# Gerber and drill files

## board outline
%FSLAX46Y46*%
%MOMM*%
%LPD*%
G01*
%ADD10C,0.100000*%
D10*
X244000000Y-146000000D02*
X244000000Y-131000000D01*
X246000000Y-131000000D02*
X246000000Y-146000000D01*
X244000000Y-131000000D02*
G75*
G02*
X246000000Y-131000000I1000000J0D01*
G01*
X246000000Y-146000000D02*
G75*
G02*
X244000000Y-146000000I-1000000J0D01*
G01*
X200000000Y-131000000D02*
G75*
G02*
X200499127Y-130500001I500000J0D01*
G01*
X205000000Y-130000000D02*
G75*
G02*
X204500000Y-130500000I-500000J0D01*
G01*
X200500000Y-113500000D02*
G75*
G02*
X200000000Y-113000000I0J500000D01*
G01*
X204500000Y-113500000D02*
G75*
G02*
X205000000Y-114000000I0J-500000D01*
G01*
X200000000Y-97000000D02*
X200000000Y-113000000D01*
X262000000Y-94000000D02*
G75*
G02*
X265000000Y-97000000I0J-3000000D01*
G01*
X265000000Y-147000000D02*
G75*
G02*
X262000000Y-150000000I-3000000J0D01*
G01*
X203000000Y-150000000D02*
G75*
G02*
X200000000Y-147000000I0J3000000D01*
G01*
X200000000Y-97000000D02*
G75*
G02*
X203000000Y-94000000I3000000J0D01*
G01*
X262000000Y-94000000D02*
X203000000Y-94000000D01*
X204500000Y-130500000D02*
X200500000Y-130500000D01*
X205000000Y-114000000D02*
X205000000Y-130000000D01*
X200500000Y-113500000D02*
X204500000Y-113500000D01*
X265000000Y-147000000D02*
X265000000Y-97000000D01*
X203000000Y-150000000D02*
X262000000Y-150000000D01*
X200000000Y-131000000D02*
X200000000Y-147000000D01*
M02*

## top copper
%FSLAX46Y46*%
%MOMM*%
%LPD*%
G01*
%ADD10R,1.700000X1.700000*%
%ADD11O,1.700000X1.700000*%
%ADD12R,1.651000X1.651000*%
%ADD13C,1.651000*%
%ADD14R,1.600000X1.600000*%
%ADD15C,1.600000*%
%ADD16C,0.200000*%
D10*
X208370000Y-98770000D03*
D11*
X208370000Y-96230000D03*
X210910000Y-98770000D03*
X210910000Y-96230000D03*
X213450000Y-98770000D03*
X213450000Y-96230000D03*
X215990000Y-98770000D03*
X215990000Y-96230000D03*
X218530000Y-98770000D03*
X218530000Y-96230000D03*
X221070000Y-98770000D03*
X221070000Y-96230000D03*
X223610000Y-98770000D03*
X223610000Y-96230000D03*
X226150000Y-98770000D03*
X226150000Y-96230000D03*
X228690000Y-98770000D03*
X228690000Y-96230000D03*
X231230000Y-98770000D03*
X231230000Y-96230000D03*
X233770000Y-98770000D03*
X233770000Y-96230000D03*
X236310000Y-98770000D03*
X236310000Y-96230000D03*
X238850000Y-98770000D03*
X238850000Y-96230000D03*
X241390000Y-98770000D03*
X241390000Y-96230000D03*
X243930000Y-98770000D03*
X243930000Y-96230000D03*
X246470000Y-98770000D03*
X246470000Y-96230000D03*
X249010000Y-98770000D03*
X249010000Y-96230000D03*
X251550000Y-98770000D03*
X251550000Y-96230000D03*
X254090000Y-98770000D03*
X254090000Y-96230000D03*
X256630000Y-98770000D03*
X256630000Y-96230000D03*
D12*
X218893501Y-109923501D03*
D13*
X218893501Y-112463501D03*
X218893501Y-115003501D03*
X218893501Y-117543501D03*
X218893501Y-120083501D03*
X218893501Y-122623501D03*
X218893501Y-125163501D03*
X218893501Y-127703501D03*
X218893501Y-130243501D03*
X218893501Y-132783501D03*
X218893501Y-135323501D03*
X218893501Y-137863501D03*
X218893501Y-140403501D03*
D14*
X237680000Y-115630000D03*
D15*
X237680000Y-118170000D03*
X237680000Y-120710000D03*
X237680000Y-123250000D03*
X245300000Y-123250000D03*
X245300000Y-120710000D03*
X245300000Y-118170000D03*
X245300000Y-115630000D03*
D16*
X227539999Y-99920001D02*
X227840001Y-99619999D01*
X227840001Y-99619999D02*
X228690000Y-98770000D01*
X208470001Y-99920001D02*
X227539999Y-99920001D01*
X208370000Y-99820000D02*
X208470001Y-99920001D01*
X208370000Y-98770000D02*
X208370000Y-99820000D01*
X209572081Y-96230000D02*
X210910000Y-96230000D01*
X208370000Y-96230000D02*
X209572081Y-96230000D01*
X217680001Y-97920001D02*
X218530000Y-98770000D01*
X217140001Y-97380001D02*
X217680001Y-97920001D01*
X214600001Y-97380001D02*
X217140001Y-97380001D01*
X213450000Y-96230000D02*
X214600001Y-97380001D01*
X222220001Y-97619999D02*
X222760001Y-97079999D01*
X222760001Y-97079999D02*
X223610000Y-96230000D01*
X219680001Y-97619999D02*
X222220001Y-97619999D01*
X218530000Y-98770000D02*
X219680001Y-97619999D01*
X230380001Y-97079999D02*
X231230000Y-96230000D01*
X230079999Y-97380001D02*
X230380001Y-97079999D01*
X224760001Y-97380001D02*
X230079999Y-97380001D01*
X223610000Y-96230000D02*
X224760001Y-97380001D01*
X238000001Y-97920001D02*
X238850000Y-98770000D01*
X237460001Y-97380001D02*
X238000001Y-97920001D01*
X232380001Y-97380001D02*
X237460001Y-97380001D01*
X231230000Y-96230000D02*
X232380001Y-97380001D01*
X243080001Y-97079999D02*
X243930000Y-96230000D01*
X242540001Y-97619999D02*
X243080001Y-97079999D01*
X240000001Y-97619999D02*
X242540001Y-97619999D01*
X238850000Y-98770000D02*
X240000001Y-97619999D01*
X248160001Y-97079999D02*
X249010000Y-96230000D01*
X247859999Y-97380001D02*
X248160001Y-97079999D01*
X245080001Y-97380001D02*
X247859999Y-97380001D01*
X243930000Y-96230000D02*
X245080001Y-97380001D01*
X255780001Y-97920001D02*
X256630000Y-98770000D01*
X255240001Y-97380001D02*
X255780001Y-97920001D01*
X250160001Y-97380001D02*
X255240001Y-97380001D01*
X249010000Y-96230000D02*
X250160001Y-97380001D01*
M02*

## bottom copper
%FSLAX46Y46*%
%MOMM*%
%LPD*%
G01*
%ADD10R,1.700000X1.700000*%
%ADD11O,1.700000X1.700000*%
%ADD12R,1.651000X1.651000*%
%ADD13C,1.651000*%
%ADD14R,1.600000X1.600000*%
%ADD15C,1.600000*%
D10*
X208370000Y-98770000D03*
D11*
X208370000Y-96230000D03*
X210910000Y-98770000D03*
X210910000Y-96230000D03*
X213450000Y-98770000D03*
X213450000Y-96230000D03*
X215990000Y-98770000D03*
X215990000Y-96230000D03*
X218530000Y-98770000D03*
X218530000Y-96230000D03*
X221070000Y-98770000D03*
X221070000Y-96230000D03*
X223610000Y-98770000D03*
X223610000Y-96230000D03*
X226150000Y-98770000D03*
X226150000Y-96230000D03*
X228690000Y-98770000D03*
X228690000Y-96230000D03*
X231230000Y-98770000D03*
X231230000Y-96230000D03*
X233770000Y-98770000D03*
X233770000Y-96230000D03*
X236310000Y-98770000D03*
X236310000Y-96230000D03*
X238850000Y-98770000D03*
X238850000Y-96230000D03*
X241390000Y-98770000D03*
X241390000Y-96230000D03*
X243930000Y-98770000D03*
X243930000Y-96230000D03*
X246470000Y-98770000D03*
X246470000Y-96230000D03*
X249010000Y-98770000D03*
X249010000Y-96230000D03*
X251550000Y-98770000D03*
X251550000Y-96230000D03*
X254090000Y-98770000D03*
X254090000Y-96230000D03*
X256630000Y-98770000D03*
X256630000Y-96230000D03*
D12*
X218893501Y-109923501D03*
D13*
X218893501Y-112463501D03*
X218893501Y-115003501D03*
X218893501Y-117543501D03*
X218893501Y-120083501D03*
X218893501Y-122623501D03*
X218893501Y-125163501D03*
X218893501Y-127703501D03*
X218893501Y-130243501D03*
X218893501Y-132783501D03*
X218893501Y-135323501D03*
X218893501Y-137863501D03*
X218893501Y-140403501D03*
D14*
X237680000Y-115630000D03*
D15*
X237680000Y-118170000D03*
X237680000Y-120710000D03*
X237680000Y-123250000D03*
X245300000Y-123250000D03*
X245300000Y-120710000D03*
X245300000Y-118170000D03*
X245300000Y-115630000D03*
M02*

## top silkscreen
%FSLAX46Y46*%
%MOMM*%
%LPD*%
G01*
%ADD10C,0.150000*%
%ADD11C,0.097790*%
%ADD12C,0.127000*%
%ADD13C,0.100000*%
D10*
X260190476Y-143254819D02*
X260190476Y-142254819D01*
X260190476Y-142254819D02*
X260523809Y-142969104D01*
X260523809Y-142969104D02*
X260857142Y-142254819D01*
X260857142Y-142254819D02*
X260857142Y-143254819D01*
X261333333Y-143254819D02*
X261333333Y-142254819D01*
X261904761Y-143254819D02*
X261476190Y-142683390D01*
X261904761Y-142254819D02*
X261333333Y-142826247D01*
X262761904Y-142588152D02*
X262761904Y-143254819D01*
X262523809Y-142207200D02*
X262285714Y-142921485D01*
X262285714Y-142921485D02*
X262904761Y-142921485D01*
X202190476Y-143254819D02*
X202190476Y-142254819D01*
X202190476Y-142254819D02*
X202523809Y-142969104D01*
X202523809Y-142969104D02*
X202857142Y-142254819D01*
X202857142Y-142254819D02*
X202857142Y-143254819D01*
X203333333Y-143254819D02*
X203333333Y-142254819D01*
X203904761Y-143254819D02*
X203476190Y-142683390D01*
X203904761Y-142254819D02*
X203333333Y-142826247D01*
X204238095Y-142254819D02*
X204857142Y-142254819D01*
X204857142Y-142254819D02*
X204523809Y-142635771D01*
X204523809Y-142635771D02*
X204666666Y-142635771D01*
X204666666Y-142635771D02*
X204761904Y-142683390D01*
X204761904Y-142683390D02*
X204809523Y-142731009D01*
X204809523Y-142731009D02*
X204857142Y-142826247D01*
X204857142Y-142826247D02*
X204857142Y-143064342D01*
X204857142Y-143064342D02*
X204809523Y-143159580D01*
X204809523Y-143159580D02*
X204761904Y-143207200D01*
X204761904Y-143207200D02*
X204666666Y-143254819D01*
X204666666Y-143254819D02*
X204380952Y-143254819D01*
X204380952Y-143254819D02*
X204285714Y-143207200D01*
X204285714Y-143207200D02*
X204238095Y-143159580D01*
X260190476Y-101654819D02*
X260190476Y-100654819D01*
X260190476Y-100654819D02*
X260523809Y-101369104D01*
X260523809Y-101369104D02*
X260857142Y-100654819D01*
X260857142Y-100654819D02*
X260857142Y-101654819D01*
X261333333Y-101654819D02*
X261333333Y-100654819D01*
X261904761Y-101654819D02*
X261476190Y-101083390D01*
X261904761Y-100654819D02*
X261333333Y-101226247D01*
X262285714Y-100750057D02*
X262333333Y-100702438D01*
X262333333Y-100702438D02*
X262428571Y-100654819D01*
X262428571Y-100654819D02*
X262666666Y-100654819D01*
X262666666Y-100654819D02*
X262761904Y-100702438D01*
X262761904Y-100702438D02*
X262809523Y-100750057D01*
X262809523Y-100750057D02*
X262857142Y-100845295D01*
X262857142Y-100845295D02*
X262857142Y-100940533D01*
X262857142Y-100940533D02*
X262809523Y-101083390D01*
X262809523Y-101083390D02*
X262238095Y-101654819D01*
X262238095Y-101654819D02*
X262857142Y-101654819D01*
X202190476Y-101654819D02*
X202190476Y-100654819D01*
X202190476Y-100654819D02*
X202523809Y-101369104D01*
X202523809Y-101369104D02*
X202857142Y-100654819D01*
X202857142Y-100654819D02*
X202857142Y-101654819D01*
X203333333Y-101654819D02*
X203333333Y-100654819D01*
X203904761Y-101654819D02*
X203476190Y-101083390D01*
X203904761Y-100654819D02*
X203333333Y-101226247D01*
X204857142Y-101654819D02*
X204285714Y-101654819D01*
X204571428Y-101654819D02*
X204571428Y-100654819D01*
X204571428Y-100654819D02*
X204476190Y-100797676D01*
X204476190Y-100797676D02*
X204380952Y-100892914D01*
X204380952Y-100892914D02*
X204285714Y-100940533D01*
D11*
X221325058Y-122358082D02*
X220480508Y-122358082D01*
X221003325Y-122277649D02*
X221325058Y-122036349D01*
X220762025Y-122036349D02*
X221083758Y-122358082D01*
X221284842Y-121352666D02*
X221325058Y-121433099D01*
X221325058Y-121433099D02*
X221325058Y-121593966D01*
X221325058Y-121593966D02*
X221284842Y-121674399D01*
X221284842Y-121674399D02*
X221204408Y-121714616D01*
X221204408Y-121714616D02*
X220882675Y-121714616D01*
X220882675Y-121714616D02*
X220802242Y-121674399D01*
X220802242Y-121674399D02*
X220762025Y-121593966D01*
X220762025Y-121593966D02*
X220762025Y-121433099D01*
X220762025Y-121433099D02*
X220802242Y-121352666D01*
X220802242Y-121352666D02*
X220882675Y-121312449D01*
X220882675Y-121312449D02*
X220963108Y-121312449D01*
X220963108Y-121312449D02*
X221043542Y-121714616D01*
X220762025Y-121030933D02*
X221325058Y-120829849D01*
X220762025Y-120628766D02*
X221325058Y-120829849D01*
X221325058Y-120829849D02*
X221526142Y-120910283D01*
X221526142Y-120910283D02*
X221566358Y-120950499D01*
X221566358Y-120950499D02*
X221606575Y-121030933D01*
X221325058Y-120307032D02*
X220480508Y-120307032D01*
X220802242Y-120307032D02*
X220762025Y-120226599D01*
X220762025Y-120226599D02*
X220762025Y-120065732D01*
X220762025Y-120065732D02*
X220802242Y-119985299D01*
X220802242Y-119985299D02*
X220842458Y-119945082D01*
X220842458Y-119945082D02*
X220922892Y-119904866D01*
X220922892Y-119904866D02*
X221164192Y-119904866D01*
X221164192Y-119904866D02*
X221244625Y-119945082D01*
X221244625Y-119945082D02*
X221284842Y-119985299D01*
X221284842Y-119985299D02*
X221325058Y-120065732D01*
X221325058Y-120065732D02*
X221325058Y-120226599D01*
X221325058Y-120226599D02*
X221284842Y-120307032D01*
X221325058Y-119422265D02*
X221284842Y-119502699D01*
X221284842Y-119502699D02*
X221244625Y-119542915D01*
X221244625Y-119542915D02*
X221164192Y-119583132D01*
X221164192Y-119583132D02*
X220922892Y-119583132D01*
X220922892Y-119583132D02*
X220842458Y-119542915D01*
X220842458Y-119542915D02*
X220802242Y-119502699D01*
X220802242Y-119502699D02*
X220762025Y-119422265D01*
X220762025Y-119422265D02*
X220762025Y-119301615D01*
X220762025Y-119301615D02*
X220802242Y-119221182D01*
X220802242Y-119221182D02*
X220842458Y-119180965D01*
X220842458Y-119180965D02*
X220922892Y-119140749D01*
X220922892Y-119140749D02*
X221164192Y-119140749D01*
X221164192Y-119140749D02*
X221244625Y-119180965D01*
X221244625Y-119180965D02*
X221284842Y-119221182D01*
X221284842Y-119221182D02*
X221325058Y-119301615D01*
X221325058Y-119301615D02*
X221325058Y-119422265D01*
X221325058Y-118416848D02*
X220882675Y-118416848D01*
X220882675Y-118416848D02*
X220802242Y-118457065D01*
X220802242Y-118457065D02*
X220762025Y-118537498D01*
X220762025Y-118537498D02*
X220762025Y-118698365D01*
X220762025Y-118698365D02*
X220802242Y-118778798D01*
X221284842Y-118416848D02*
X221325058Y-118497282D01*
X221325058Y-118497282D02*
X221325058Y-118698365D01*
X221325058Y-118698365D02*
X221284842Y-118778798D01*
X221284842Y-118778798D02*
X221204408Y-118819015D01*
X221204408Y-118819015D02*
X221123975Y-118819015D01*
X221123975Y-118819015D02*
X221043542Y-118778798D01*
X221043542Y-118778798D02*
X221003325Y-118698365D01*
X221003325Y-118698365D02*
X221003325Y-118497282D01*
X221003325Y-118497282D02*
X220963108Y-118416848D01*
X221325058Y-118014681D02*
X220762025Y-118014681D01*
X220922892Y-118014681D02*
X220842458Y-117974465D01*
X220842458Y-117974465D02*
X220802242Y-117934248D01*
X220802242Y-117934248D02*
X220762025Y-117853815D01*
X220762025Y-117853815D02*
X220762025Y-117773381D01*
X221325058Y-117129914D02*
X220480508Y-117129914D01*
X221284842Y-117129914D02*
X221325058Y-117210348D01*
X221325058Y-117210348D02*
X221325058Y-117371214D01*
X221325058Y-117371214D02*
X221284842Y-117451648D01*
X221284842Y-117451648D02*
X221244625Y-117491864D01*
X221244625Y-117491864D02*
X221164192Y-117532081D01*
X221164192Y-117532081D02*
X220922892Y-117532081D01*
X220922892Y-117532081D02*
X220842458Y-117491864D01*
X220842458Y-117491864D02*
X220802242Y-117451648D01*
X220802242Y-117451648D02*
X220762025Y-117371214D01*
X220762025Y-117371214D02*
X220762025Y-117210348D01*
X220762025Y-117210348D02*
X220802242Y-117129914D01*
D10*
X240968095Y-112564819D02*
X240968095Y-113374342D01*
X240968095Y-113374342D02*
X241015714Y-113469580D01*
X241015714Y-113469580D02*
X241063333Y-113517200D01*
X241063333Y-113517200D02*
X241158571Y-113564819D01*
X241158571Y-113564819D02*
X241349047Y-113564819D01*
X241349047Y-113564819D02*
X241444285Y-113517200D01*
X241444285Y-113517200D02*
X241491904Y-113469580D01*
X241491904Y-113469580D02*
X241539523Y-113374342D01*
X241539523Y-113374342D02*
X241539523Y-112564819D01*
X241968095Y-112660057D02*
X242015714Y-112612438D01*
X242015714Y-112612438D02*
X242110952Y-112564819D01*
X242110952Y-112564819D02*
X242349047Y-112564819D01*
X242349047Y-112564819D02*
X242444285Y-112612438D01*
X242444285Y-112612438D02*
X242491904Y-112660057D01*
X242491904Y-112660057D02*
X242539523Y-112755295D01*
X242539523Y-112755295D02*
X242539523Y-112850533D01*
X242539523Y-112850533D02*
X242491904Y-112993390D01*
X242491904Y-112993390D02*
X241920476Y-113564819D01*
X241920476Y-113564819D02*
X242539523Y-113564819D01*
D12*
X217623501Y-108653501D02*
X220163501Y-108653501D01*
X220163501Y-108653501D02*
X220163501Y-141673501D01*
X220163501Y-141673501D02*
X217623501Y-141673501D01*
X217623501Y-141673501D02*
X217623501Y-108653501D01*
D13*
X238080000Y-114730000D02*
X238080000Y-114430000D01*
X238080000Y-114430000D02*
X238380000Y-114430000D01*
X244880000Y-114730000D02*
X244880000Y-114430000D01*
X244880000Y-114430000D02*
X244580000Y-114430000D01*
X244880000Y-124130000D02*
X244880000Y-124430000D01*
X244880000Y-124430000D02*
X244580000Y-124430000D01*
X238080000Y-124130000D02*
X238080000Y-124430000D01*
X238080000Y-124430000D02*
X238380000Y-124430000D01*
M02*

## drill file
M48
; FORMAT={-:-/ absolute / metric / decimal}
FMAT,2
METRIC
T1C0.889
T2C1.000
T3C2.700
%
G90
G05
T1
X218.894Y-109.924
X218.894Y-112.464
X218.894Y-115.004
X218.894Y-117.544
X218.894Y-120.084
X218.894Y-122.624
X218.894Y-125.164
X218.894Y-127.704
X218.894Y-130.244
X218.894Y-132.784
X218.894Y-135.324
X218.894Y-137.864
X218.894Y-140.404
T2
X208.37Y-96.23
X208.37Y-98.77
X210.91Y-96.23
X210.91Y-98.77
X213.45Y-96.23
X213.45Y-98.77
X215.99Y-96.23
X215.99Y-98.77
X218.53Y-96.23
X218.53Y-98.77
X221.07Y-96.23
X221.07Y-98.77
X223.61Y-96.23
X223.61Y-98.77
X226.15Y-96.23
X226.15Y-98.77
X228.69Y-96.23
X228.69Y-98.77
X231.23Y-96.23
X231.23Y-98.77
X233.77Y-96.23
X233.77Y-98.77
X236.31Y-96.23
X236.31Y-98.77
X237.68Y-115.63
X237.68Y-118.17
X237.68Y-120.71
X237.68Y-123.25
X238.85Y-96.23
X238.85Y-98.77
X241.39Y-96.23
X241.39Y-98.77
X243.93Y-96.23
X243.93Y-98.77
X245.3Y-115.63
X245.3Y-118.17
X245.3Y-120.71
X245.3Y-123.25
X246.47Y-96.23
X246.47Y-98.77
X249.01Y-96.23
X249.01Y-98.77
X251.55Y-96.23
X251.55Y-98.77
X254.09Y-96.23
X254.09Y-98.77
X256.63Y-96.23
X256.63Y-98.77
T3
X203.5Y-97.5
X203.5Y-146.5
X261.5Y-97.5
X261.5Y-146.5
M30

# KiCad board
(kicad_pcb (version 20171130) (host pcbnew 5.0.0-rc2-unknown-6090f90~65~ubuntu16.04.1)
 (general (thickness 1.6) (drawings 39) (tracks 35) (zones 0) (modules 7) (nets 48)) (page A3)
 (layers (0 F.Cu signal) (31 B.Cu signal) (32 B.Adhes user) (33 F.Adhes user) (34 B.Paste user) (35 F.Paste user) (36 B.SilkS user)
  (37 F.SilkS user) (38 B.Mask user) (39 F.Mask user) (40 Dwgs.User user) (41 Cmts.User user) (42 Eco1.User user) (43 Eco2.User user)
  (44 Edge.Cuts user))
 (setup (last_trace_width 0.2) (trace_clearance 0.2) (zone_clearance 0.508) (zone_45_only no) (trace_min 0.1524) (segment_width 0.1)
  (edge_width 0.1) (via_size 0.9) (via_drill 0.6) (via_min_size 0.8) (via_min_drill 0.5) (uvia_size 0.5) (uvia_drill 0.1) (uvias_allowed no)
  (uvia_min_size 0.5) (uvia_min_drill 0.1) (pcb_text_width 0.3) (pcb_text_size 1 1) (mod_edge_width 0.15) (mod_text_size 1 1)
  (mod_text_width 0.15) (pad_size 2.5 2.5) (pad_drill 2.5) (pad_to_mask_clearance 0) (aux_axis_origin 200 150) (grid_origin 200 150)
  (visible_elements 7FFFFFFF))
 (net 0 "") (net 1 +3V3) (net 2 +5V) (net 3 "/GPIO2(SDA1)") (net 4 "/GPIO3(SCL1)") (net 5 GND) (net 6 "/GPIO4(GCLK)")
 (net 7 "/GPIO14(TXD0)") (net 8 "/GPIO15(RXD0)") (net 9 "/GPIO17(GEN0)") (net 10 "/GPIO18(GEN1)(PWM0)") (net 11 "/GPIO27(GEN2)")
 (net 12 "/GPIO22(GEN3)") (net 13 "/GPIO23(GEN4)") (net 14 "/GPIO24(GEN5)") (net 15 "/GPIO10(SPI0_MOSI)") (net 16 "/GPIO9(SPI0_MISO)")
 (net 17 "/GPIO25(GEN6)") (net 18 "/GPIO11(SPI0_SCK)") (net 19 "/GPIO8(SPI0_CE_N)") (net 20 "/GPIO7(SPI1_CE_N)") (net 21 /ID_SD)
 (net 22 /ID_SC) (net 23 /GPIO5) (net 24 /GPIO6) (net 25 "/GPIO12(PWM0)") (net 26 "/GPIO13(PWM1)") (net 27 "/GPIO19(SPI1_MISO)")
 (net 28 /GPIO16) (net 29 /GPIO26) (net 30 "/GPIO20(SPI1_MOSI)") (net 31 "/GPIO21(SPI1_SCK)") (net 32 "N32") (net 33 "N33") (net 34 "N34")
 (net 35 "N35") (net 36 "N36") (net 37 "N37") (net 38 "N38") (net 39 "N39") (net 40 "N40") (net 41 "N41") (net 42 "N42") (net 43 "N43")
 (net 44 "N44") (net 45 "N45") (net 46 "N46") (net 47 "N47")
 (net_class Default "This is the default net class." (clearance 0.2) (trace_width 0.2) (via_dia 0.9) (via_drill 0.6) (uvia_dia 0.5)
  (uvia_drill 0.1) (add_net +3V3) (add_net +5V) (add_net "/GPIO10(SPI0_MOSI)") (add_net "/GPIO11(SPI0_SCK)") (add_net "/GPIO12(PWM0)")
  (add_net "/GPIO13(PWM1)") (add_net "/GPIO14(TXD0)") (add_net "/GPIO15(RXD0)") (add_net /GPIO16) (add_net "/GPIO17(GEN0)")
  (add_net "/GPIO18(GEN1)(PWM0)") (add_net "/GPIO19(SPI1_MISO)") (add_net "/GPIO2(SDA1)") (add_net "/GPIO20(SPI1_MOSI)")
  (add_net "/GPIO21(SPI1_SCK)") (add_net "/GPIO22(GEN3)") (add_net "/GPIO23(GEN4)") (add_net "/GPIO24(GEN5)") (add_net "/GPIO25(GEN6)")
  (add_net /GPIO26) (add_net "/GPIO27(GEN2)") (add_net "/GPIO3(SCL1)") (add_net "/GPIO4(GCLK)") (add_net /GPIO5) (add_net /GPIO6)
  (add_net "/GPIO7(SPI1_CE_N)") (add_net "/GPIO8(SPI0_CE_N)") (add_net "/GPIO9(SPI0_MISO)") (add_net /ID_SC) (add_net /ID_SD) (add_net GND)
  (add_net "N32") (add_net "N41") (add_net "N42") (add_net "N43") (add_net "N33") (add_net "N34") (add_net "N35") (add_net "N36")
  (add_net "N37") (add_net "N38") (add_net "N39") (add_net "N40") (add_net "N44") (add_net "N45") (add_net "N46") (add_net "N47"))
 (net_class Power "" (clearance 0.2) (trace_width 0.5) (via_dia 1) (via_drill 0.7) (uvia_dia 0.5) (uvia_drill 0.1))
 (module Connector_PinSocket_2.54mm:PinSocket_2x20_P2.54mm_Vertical (layer B.Cu) (at 208.37 98.77 270)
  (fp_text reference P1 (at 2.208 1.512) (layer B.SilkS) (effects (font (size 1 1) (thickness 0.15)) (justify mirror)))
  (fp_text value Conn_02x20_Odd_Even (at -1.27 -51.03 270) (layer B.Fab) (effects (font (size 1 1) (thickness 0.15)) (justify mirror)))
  (pad 1 thru_hole rect (at 0 0 270) (size 1.7 1.7) (drill 1) (layers *.Cu *.Mask) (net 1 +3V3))
  (pad 2 thru_hole oval (at -2.54 0 270) (size 1.7 1.7) (drill 1) (layers *.Cu *.Mask) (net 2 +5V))
  (pad 3 thru_hole oval (at 0 -2.54 270) (size 1.7 1.7) (drill 1) (layers *.Cu *.Mask) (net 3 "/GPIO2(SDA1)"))
  (pad 4 thru_hole oval (at -2.54 -2.54 270) (size 1.7 1.7) (drill 1) (layers *.Cu *.Mask) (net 2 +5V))
  (pad 5 thru_hole oval (at 0 -5.08 270) (size 1.7 1.7) (drill 1) (layers *.Cu *.Mask) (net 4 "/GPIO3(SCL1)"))
  (pad 6 thru_hole oval (at -2.54 -5.08 270) (size 1.7 1.7) (drill 1) (layers *.Cu *.Mask) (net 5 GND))
  (pad 7 thru_hole oval (at 0 -7.62 270) (size 1.7 1.7) (drill 1) (layers *.Cu *.Mask) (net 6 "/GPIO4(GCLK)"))
  (pad 8 thru_hole oval (at -2.54 -7.62 270) (size 1.7 1.7) (drill 1) (layers *.Cu *.Mask) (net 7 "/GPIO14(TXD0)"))
  (pad 9 thru_hole oval (at 0 -10.16 270) (size 1.7 1.7) (drill 1) (layers *.Cu *.Mask) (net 5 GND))
  (pad 10 thru_hole oval (at -2.54 -10.16 270) (size 1.7 1.7) (drill 1) (layers *.Cu *.Mask) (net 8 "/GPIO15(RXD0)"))
  (pad 11 thru_hole oval (at 0 -12.7 270) (size 1.7 1.7) (drill 1) (layers *.Cu *.Mask) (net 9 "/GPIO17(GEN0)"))
  (pad 12 thru_hole oval (at -2.54 -12.7 270) (size 1.7 1.7) (drill 1) (layers *.Cu *.Mask) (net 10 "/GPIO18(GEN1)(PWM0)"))
  (pad 13 thru_hole oval (at 0 -15.24 270) (size 1.7 1.7) (drill 1) (layers *.Cu *.Mask) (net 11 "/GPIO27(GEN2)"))
  (pad 14 thru_hole oval (at -2.54 -15.24 270) (size 1.7 1.7) (drill 1) (layers *.Cu *.Mask) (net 5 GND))
  (pad 15 thru_hole oval (at 0 -17.78 270) (size 1.7 1.7) (drill 1) (layers *.Cu *.Mask) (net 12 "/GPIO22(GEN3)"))
  (pad 16 thru_hole oval (at -2.54 -17.78 270) (size 1.7 1.7) (drill 1) (layers *.Cu *.Mask) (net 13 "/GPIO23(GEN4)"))
  (pad 17 thru_hole oval (at 0 -20.32 270) (size 1.7 1.7) (drill 1) (layers *.Cu *.Mask) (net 1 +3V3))
  (pad 18 thru_hole oval (at -2.54 -20.32 270) (size 1.7 1.7) (drill 1) (layers *.Cu *.Mask) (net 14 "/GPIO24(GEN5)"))
  (pad 19 thru_hole oval (at 0 -22.86 270) (size 1.7 1.7) (drill 1) (layers *.Cu *.Mask) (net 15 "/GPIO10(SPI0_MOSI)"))
  (pad 20 thru_hole oval (at -2.54 -22.86 270) (size 1.7 1.7) (drill 1) (layers *.Cu *.Mask) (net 5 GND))
  (pad 21 thru_hole oval (at 0 -25.4 270) (size 1.7 1.7) (drill 1) (layers *.Cu *.Mask) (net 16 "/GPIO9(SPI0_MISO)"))
  (pad 22 thru_hole oval (at -2.54 -25.4 270) (size 1.7 1.7) (drill 1) (layers *.Cu *.Mask) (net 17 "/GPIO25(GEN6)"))
  (pad 23 thru_hole oval (at 0 -27.94 270) (size 1.7 1.7) (drill 1) (layers *.Cu *.Mask) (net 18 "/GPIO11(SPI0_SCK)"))
  (pad 24 thru_hole oval (at -2.54 -27.94 270) (size 1.7 1.7) (drill 1) (layers *.Cu *.Mask) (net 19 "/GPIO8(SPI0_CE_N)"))
  (pad 25 thru_hole oval (at 0 -30.48 270) (size 1.7 1.7) (drill 1) (layers *.Cu *.Mask) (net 5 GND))
  (pad 26 thru_hole oval (at -2.54 -30.48 270) (size 1.7 1.7) (drill 1) (layers *.Cu *.Mask) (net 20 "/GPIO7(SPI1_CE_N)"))
  (pad 27 thru_hole oval (at 0 -33.02 270) (size 1.7 1.7) (drill 1) (layers *.Cu *.Mask) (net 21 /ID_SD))
  (pad 28 thru_hole oval (at -2.54 -33.02 270) (size 1.7 1.7) (drill 1) (layers *.Cu *.Mask) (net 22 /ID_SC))
  (pad 29 thru_hole oval (at 0 -35.56 270) (size 1.7 1.7) (drill 1) (layers *.Cu *.Mask) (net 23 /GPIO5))
  (pad 30 thru_hole oval (at -2.54 -35.56 270) (size 1.7 1.7) (drill 1) (layers *.Cu *.Mask) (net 5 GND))
  (pad 31 thru_hole oval (at 0 -38.1 270) (size 1.7 1.7) (drill 1) (layers *.Cu *.Mask) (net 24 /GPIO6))
  (pad 32 thru_hole oval (at -2.54 -38.1 270) (size 1.7 1.7) (drill 1) (layers *.Cu *.Mask) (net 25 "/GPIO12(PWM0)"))
  (pad 33 thru_hole oval (at 0 -40.64 270) (size 1.7 1.7) (drill 1) (layers *.Cu *.Mask) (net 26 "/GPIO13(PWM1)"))
  (pad 34 thru_hole oval (at -2.54 -40.64 270) (size 1.7 1.7) (drill 1) (layers *.Cu *.Mask) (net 5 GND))
  (pad 35 thru_hole oval (at 0 -43.18 270) (size 1.7 1.7) (drill 1) (layers *.Cu *.Mask) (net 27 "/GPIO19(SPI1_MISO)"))
  (pad 36 thru_hole oval (at -2.54 -43.18 270) (size 1.7 1.7) (drill 1) (layers *.Cu *.Mask) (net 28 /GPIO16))
  (pad 37 thru_hole oval (at 0 -45.72 270) (size 1.7 1.7) (drill 1) (layers *.Cu *.Mask) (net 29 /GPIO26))
  (pad 38 thru_hole oval (at -2.54 -45.72 270) (size 1.7 1.7) (drill 1) (layers *.Cu *.Mask) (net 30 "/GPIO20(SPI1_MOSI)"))
  (pad 39 thru_hole oval (at 0 -48.26 270) (size 1.7 1.7) (drill 1) (layers *.Cu *.Mask) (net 5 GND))
  (pad 40 thru_hole oval (at -2.54 -48.26 270) (size 1.7 1.7) (drill 1) (layers *.Cu *.Mask) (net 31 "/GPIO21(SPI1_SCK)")))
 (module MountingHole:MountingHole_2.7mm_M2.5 (layer F.Cu) (at 261.5 146.5)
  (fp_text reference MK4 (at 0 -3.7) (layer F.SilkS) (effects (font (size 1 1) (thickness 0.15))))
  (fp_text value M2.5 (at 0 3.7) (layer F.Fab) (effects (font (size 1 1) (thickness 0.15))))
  (pad 1 np_thru_hole circle (at 0 0) (size 2.7 2.7) (drill 2.7) (layers *.Cu *.Mask)))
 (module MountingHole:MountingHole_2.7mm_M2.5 (layer F.Cu) (at 203.5 146.5)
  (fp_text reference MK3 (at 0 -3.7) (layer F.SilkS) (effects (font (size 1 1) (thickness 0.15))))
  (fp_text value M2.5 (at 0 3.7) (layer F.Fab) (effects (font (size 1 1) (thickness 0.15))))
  (pad 1 np_thru_hole circle (at 0 0) (size 2.7 2.7) (drill 2.7) (layers *.Cu *.Mask)))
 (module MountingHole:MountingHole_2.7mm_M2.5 (layer F.Cu) (at 261.5 97.5 180)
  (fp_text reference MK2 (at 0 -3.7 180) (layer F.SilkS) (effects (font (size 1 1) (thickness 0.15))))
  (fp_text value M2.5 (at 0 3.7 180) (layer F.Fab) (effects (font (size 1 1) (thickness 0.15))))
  (pad 1 np_thru_hole circle (at 0 0 180) (size 2.7 2.7) (drill 2.7) (layers *.Cu *.Mask)))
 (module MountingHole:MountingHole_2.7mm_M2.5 (layer F.Cu) (at 203.5 97.5 180)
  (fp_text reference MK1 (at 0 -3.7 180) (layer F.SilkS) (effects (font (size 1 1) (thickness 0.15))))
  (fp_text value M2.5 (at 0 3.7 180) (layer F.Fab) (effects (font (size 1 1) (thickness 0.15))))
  (pad 1 np_thru_hole circle (at 0 0 180) (size 2.7 2.7) (drill 2.7) (layers *.Cu *.Mask)))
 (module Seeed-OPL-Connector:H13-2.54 (layer F.Cu) (at 218.893501 125.163501)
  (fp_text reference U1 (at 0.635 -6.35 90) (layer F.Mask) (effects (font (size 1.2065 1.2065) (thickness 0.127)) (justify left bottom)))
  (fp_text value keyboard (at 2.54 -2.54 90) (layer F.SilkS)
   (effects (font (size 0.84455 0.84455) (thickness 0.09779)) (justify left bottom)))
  (fp_line (start -1.27 -16.51) (end 1.27 -16.51) (layer F.SilkS) (width 0.127))
  (fp_line (start 1.27 -16.51) (end 1.27 16.51) (layer F.SilkS) (width 0.127))
  (fp_line (start 1.27 16.51) (end -1.27 16.51) (layer F.SilkS) (width 0.127))
  (fp_line (start -1.27 16.51) (end -1.27 -16.51) (layer F.SilkS) (width 0.127))
  (pad 1 thru_hole rect (at 0 -15.24) (size 1.651 1.651) (drill 0.889) (layers *.Cu *.Mask) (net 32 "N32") (solder_mask_margin 0.1016))
  (pad 2 thru_hole circle (at 0 -12.7) (size 1.651 1.651) (drill 0.889) (layers *.Cu *.Mask) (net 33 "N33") (solder_mask_margin 0.1016))
  (pad 3 thru_hole circle (at 0 -10.16) (size 1.651 1.651) (drill 0.889) (layers *.Cu *.Mask) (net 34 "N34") (solder_mask_margin 0.1016))
  (pad 4 thru_hole circle (at 0 -7.62) (size 1.651 1.651) (drill 0.889) (layers *.Cu *.Mask) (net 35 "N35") (solder_mask_margin 0.1016))
  (pad 5 thru_hole circle (at 0 -5.08) (size 1.651 1.651) (drill 0.889) (layers *.Cu *.Mask) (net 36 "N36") (solder_mask_margin 0.1016))
  (pad 6 thru_hole circle (at 0 -2.54) (size 1.651 1.651) (drill 0.889) (layers *.Cu *.Mask) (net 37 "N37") (solder_mask_margin 0.1016))
  (pad 7 thru_hole circle (at 0 0) (size 1.651 1.651) (drill 0.889) (layers *.Cu *.Mask) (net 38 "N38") (solder_mask_margin 0.1016))
  (pad 8 thru_hole circle (at 0 2.54) (size 1.651 1.651) (drill 0.889) (layers *.Cu *.Mask) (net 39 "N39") (solder_mask_margin 0.1016))
  (pad 9 thru_hole circle (at 0 5.08) (size 1.651 1.651) (drill 0.889) (layers *.Cu *.Mask) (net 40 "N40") (solder_mask_margin 0.1016))
  (pad 10 thru_hole circle (at 0 7.62) (size 1.651 1.651) (drill 0.889) (layers *.Cu *.Mask) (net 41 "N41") (solder_mask_margin 0.1016))
  (pad 11 thru_hole circle (at 0 10.16) (size 1.651 1.651) (drill 0.889) (layers *.Cu *.Mask) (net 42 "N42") (solder_mask_margin 0.1016))
  (pad 12 thru_hole circle (at 0 12.7) (size 1.651 1.651) (drill 0.889) (layers *.Cu *.Mask) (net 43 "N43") (solder_mask_margin 0.1016))
  (pad 13 thru_hole circle (at 0 15.24) (size 1.651 1.651) (drill 0.889) (layers *.Cu *.Mask) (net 5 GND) (solder_mask_margin 0.1016)))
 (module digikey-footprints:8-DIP (layer F.Cu) (at 237.68 115.63)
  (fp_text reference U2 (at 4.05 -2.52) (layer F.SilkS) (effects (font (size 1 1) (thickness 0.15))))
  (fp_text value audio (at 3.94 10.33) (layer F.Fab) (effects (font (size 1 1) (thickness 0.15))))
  (fp_line (start 0.4 -0.9) (end 0.4 -1.2) (layer F.SilkS) (width 0.1))
  (fp_line (start 0.4 -1.2) (end 0.7 -1.2) (layer F.SilkS) (width 0.1))
  (fp_line (start 7.2 -0.9) (end 7.2 -1.2) (layer F.SilkS) (width 0.1))
  (fp_line (start 7.2 -1.2) (end 6.9 -1.2) (layer F.SilkS) (width 0.1))
  (fp_line (start 7.2 8.5) (end 7.2 8.8) (layer F.SilkS) (width 0.1))
  (fp_line (start 7.2 8.8) (end 6.9 8.8) (layer F.SilkS) (width 0.1))
  (fp_line (start 0.4 8.5) (end 0.4 8.8) (layer F.SilkS) (width 0.1))
  (fp_line (start 0.4 8.8) (end 0.7 8.8) (layer F.SilkS) (width 0.1))
  (pad 1 thru_hole rect (at 0 0) (size 1.6 1.6) (drill 1) (layers *.Cu *.Mask) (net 26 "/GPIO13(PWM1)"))
  (pad 2 thru_hole circle (at 0 2.54) (size 1.6 1.6) (drill 1) (layers *.Cu *.Mask) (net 2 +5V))
  (pad 3 thru_hole circle (at 0 5.08) (size 1.6 1.6) (drill 1) (layers *.Cu *.Mask) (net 5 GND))
  (pad 4 thru_hole circle (at 0 7.62) (size 1.6 1.6) (drill 1) (layers *.Cu *.Mask) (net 10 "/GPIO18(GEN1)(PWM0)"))
  (pad 5 thru_hole circle (at 7.62 7.62) (size 1.6 1.6) (drill 1) (layers *.Cu *.Mask) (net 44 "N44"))
  (pad 6 thru_hole circle (at 7.62 5.08) (size 1.6 1.6) (drill 1) (layers *.Cu *.Mask) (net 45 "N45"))
  (pad 7 thru_hole circle (at 7.62 2.54) (size 1.6 1.6) (drill 1) (layers *.Cu *.Mask) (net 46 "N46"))
  (pad 8 thru_hole circle (at 7.62 0) (size 1.6 1.6) (drill 1) (layers *.Cu *.Mask) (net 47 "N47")))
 (gr_line (start 244 146) (end 244 131) (layer Edge.Cuts) (width 0.1))
 (gr_line (start 246 131) (end 246 146) (layer Edge.Cuts) (width 0.1))
 (gr_arc (start 245 131) (end 244 131) (angle 180) (layer Edge.Cuts) (width 0.1))
 (gr_arc (start 245 146) (end 246 146) (angle 180) (layer Edge.Cuts) (width 0.1))
 (gr_arc (start 200.5 131) (end 200 131) (angle 89.9) (layer Edge.Cuts) (width 0.1))
 (gr_arc (start 204.5 130) (end 205 130) (angle 90) (layer Edge.Cuts) (width 0.1))
 (gr_arc (start 200.5 113) (end 200.5 113.5) (angle 90) (layer Edge.Cuts) (width 0.1))
 (gr_arc (start 204.5 114) (end 204.5 113.5) (angle 90) (layer Edge.Cuts) (width 0.1))
 (gr_line (start 200 97) (end 200 113) (layer Edge.Cuts) (width 0.1))
 (gr_arc (start 262 97) (end 262 94) (angle 90) (layer Edge.Cuts) (width 0.1))
 (gr_arc (start 262 147) (end 265 147) (angle 90) (layer Edge.Cuts) (width 0.1))
 (gr_arc (start 203 147) (end 203 150) (angle 90) (layer Edge.Cuts) (width 0.1))
 (gr_arc (start 203 97) (end 200 97) (angle 90) (layer Edge.Cuts) (width 0.1))
 (gr_line (start 262 94) (end 203 94) (layer Edge.Cuts) (width 0.1))
 (gr_line (start 204.5 130.5) (end 200.5 130.5) (layer Edge.Cuts) (width 0.1))
 (gr_line (start 205 114) (end 205 130) (layer Edge.Cuts) (width 0.1))
 (gr_line (start 200.5 113.5) (end 204.5 113.5) (layer Edge.Cuts) (width 0.1))
 (gr_line (start 265 147) (end 265 97) (layer Edge.Cuts) (width 0.1))
 (gr_line (start 203 150) (end 262 150) (layer Edge.Cuts) (width 0.1))
 (gr_line (start 200 131) (end 200 147) (layer Edge.Cuts) (width 0.1))
 (segment (start 227.539999 99.920001) (end 227.840001 99.619999) (width 0.2) (layer F.Cu) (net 1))
 (segment (start 227.840001 99.619999) (end 228.69 98.77) (width 0.2) (layer F.Cu) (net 1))
 (segment (start 208.470001 99.920001) (end 227.539999 99.920001) (width 0.2) (layer F.Cu) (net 1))
 (segment (start 208.37 99.82) (end 208.470001 99.920001) (width 0.2) (layer F.Cu) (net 1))
 (segment (start 208.37 98.77) (end 208.37 99.82) (width 0.2) (layer F.Cu) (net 1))
 (segment (start 209.572081 96.23) (end 210.91 96.23) (width 0.2) (layer F.Cu) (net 2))
 (segment (start 208.37 96.23) (end 209.572081 96.23) (width 0.2) (layer F.Cu) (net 2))
 (segment (start 217.680001 97.920001) (end 218.53 98.77) (width 0.2) (layer F.Cu) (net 5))
 (segment (start 217.140001 97.380001) (end 217.680001 97.920001) (width 0.2) (layer F.Cu) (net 5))
 (segment (start 214.600001 97.380001) (end 217.140001 97.380001) (width 0.2) (layer F.Cu) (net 5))
 (segment (start 213.45 96.23) (end 214.600001 97.380001) (width 0.2) (layer F.Cu) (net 5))
 (segment (start 222.220001 97.619999) (end 222.760001 97.079999) (width 0.2) (layer F.Cu) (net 5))
 (segment (start 222.760001 97.079999) (end 223.61 96.23) (width 0.2) (layer F.Cu) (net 5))
 (segment (start 219.680001 97.619999) (end 222.220001 97.619999) (width 0.2) (layer F.Cu) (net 5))
 (segment (start 218.53 98.77) (end 219.680001 97.619999) (width 0.2) (layer F.Cu) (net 5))
 (segment (start 230.380001 97.079999) (end 231.23 96.23) (width 0.2) (layer F.Cu) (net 5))
 (segment (start 230.079999 97.380001) (end 230.380001 97.079999) (width 0.2) (layer F.Cu) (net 5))
 (segment (start 224.760001 97.380001) (end 230.079999 97.380001) (width 0.2) (layer F.Cu) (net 5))
 (segment (start 223.61 96.23) (end 224.760001 97.380001) (width 0.2) (layer F.Cu) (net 5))
 (segment (start 238.000001 97.920001) (end 238.85 98.77) (width 0.2) (layer F.Cu) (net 5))
 (segment (start 237.460001 97.380001) (end 238.000001 97.920001) (width 0.2) (layer F.Cu) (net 5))
 (segment (start 232.380001 97.380001) (end 237.460001 97.380001) (width 0.2) (layer F.Cu) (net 5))
 (segment (start 231.23 96.23) (end 232.380001 97.380001) (width 0.2) (layer F.Cu) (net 5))
 (segment (start 243.080001 97.079999) (end 243.93 96.23) (width 0.2) (layer F.Cu) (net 5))
 (segment (start 242.540001 97.619999) (end 243.080001 97.079999) (width 0.2) (layer F.Cu) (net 5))
 (segment (start 240.000001 97.619999) (end 242.540001 97.619999) (width 0.2) (layer F.Cu) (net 5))
 (segment (start 238.85 98.77) (end 240.000001 97.619999) (width 0.2) (layer F.Cu) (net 5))
 (segment (start 248.160001 97.079999) (end 249.01 96.23) (width 0.2) (layer F.Cu) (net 5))
 (segment (start 247.859999 97.380001) (end 248.160001 97.079999) (width 0.2) (layer F.Cu) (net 5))
 (segment (start 245.080001 97.380001) (end 247.859999 97.380001) (width 0.2) (layer F.Cu) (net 5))
 (segment (start 243.93 96.23) (end 245.080001 97.380001) (width 0.2) (layer F.Cu) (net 5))
 (segment (start 255.780001 97.920001) (end 256.63 98.77) (width 0.2) (layer F.Cu) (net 5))
 (segment (start 255.240001 97.380001) (end 255.780001 97.920001) (width 0.2) (layer F.Cu) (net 5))
 (segment (start 250.160001 97.380001) (end 255.240001 97.380001) (width 0.2) (layer F.Cu) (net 5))
 (segment (start 249.01 96.23) (end 250.160001 97.380001) (width 0.2) (layer F.Cu) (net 5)))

